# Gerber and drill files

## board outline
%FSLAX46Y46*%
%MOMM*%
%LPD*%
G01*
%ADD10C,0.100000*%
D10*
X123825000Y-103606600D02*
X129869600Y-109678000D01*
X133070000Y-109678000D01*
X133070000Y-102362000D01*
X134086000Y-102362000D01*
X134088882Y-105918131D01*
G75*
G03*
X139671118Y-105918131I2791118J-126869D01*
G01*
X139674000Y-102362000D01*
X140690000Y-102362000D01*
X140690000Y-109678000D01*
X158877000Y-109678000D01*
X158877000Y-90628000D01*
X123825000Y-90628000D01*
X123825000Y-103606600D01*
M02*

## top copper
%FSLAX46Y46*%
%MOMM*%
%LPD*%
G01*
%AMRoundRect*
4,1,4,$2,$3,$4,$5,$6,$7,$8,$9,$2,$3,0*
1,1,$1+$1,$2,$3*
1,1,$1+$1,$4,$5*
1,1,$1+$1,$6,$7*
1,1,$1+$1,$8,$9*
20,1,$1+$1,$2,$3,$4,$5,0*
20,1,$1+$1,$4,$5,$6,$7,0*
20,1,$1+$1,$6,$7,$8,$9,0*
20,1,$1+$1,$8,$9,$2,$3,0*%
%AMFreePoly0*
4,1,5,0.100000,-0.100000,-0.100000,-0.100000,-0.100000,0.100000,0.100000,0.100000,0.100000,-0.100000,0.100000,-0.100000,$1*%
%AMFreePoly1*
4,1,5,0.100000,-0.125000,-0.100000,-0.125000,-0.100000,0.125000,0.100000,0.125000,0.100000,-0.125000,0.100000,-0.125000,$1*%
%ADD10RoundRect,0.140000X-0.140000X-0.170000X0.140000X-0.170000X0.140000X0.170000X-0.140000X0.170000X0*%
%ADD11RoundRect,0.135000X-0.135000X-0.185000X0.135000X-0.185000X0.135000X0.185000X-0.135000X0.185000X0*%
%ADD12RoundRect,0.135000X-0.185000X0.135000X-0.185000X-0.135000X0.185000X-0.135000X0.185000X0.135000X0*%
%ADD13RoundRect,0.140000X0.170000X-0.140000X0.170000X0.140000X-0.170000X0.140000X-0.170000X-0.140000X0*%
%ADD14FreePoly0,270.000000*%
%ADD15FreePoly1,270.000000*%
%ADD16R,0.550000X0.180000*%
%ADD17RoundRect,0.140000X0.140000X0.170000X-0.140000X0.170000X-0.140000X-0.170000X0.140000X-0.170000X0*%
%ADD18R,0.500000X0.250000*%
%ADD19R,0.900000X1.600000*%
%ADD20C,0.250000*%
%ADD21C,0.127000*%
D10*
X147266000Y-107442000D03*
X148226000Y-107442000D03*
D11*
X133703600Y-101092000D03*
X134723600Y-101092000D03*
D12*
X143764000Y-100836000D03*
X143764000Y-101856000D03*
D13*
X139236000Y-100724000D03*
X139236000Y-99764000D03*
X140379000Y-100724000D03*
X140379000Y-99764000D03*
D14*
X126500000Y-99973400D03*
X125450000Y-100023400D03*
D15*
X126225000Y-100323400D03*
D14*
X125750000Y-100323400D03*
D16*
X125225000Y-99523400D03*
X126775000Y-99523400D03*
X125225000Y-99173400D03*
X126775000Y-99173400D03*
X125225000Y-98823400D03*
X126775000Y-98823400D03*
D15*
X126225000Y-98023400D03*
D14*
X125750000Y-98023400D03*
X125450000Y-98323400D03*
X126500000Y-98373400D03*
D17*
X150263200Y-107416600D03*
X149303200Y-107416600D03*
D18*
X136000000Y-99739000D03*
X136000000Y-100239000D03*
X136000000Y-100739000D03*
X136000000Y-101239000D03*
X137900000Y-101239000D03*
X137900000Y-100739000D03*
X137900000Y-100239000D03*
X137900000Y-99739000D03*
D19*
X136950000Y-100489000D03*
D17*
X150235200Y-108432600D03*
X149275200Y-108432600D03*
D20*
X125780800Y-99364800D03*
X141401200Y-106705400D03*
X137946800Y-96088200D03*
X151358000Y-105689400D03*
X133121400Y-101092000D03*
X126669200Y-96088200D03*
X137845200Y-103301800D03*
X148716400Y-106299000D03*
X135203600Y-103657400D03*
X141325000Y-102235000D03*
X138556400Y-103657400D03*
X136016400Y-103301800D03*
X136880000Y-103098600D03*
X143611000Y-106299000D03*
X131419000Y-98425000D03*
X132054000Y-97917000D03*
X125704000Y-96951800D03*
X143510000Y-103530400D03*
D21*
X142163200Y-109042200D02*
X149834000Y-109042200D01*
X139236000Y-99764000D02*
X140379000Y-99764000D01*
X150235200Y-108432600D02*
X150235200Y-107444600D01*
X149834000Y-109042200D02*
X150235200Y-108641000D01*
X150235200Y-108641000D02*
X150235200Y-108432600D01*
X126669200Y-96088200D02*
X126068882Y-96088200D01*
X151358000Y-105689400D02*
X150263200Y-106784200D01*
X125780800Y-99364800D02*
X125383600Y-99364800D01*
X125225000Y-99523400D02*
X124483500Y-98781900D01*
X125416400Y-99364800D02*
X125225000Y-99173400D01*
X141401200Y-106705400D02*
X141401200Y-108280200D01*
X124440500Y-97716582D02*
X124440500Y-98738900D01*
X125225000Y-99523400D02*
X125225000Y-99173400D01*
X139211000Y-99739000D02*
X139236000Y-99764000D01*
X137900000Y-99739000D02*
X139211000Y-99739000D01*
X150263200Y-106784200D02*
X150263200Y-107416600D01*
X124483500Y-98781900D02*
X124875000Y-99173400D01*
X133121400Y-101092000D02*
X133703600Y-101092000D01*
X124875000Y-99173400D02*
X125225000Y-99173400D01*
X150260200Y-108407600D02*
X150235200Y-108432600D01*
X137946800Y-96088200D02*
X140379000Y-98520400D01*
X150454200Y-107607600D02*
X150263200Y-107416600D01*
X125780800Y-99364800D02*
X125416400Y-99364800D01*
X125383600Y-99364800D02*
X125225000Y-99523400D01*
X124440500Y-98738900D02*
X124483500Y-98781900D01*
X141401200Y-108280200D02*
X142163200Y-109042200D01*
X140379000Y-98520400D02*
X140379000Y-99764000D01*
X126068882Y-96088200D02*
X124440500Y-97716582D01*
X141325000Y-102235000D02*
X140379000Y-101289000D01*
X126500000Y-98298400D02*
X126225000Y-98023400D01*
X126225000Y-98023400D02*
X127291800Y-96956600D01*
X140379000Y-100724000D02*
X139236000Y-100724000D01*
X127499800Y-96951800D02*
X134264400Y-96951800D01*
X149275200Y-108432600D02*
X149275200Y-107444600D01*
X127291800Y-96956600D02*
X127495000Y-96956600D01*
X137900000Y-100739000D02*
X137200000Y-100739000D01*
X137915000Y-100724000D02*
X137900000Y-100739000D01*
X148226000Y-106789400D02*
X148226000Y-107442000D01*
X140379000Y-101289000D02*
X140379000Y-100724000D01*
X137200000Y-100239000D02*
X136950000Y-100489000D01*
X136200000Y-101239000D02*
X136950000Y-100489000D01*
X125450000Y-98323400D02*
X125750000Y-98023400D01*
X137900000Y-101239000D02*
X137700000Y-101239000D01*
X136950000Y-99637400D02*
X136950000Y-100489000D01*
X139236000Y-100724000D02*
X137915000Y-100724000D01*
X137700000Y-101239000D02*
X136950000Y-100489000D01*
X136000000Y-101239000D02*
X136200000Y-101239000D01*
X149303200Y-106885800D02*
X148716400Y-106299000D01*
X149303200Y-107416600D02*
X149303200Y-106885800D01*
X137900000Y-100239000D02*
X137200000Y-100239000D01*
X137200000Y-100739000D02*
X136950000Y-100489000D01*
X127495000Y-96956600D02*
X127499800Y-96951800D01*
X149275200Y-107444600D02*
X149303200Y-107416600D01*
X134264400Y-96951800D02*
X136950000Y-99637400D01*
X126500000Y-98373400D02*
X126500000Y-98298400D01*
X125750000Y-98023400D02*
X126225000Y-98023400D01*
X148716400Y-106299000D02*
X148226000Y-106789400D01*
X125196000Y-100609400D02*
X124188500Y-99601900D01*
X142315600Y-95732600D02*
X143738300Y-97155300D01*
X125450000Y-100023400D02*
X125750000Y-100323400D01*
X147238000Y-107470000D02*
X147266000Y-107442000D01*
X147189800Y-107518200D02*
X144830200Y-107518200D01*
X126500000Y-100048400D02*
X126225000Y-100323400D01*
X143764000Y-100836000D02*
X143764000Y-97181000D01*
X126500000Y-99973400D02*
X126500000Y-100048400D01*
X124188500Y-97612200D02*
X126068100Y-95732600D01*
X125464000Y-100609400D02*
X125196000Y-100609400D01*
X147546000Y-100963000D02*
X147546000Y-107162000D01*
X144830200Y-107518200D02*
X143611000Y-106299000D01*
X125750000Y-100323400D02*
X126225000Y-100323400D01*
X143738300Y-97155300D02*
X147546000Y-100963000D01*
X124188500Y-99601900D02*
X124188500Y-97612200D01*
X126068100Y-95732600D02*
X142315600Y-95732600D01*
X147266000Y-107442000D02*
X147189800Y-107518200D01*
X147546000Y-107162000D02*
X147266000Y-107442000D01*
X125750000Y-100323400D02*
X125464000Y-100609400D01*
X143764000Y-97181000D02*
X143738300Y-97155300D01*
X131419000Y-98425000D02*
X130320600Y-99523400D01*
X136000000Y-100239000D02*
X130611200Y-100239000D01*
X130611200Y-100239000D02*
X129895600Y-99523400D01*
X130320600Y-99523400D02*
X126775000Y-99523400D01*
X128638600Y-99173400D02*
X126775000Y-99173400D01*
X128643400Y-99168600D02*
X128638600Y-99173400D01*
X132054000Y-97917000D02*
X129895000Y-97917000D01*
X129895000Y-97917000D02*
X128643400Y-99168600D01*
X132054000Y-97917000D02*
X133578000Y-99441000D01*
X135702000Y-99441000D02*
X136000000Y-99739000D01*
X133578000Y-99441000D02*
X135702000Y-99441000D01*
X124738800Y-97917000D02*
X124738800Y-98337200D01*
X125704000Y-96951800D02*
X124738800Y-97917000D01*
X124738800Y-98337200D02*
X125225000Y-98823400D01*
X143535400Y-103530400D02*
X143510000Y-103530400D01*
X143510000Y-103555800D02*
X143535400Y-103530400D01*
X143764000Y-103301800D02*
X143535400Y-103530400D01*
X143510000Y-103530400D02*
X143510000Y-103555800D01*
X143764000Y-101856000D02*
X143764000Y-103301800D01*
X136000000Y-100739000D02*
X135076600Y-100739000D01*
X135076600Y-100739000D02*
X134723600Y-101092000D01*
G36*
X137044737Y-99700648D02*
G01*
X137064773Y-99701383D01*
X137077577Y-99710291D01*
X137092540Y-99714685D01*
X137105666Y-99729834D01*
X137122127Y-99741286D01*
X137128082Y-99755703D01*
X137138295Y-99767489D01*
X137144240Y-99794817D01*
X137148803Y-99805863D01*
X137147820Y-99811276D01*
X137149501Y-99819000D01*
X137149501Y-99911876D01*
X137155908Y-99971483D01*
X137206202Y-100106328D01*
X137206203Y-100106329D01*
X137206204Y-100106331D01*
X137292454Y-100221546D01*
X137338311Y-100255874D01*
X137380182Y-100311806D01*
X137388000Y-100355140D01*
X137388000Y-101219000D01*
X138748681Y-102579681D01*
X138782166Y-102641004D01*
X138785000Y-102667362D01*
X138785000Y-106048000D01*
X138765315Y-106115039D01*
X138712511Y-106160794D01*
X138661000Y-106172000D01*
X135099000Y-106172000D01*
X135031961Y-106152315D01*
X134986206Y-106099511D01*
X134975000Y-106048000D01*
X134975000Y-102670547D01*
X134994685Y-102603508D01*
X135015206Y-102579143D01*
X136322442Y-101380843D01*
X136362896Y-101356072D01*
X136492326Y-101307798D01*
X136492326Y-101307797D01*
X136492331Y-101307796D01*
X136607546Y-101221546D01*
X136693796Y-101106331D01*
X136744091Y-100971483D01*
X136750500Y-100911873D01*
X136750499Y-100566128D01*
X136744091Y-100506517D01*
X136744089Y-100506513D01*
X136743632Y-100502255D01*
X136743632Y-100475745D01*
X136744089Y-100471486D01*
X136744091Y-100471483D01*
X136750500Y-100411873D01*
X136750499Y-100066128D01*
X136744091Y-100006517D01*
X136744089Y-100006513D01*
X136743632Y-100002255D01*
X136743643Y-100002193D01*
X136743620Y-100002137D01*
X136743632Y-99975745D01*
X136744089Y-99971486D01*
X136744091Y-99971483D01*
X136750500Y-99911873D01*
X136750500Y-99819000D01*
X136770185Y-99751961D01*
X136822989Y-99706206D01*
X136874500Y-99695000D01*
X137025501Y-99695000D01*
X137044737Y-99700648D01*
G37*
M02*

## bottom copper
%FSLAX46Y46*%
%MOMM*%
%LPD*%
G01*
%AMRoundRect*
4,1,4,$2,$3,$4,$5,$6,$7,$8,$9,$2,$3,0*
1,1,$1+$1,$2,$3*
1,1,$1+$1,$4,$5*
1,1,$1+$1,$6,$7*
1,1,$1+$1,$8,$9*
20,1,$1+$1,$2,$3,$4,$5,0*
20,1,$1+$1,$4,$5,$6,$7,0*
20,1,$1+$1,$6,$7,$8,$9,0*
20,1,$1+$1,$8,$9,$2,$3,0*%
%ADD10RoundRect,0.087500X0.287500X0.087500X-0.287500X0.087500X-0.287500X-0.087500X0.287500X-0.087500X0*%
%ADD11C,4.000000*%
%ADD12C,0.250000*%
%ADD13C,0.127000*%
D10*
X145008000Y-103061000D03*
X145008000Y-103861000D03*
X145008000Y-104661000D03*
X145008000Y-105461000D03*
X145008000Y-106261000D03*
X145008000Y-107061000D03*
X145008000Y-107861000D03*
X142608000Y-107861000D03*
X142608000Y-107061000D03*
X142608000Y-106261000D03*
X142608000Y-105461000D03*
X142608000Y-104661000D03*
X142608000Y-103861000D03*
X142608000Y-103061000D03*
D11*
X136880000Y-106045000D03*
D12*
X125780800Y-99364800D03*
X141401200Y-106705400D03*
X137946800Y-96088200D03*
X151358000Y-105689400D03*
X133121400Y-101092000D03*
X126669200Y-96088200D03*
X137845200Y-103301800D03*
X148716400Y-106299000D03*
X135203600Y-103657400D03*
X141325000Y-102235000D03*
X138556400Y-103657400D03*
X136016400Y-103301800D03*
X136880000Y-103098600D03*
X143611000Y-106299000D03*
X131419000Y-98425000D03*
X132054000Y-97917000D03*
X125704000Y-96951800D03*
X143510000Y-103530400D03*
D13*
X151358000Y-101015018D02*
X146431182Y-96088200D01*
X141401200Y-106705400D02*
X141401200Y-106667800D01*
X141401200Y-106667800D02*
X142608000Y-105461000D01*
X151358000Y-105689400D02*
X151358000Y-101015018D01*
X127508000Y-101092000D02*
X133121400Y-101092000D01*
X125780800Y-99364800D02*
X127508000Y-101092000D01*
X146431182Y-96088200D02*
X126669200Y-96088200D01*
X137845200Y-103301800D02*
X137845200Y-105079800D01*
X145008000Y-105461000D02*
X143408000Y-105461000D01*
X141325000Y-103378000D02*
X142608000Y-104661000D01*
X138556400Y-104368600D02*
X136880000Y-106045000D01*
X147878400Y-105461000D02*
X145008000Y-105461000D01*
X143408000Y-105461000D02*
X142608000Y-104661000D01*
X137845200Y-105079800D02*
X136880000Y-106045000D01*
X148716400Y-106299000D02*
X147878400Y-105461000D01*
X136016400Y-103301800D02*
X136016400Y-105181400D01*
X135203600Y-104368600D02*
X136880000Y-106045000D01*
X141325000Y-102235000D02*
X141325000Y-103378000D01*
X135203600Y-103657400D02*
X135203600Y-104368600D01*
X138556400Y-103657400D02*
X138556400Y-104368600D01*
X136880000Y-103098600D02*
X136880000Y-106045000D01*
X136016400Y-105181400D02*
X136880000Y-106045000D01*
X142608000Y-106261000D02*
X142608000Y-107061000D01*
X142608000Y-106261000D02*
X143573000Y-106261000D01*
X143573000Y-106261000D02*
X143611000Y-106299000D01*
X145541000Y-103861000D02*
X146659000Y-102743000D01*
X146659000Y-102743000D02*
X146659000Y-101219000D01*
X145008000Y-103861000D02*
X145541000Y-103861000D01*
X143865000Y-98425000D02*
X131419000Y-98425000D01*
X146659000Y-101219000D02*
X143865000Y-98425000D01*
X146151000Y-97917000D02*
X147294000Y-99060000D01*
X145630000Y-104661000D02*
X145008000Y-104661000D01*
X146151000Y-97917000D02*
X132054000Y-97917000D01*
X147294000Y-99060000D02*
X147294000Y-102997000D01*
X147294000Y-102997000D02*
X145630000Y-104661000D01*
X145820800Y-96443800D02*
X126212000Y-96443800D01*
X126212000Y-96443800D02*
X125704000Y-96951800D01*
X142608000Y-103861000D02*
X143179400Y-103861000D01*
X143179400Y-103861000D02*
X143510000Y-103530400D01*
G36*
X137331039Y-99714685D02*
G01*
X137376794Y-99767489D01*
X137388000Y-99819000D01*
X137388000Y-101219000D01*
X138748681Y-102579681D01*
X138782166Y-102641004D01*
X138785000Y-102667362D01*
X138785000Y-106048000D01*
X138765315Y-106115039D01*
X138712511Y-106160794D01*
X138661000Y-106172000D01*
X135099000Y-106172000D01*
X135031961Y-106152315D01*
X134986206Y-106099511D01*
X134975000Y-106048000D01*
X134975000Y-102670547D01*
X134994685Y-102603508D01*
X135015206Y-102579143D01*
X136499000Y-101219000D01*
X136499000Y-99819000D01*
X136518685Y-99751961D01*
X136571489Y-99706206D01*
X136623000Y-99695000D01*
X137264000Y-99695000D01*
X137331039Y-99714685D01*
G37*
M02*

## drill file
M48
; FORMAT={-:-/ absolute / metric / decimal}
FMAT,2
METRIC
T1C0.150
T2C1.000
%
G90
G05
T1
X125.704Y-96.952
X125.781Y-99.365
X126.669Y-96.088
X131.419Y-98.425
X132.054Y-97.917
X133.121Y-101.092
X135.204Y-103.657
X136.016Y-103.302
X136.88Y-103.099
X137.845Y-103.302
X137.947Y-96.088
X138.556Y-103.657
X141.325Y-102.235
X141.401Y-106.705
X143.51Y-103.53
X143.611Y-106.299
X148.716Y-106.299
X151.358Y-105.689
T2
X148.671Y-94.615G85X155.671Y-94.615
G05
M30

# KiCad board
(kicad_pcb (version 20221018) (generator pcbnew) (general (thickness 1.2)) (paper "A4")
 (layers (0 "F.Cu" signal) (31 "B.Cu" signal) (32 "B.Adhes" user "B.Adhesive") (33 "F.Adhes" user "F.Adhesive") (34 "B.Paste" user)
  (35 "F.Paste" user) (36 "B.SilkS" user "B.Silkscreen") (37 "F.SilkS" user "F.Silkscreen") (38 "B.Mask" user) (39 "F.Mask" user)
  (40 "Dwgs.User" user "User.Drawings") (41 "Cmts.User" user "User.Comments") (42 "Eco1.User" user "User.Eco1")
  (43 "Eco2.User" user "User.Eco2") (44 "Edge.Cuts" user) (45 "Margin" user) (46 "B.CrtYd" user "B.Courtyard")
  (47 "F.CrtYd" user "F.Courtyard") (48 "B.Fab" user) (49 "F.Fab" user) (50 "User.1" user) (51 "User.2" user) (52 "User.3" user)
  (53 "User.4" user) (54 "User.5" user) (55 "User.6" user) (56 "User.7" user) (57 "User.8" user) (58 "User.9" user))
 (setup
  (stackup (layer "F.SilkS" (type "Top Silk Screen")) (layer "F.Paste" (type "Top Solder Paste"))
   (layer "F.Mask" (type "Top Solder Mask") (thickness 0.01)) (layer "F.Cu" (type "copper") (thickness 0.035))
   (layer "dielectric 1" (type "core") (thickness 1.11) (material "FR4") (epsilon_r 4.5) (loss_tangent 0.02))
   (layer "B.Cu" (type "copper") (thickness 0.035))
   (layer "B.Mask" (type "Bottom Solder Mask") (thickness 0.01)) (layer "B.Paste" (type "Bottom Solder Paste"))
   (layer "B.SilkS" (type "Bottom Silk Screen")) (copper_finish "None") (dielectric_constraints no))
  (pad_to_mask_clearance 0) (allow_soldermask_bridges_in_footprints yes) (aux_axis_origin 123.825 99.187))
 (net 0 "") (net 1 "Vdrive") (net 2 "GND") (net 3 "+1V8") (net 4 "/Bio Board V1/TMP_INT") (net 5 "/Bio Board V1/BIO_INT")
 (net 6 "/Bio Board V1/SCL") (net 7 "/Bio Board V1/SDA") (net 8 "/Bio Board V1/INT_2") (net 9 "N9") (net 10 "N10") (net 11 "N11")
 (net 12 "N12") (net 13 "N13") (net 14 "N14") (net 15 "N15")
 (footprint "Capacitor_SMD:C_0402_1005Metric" (layer "F.Cu") (at 147.746 107.442)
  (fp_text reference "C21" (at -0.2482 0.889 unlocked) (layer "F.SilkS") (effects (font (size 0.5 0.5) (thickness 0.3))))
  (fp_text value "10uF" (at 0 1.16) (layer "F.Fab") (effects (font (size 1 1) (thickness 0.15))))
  (pad "1" smd roundrect (at -0.48 0) (size 0.56 0.62) (layers "F.Cu" "F.Paste" "F.Mask") (roundrect_rratio 0.25) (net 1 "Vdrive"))
  (pad "2" smd roundrect (at 0.48 0) (size 0.56 0.62) (layers "F.Cu" "F.Paste" "F.Mask") (roundrect_rratio 0.25) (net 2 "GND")))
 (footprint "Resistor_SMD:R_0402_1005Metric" (layer "F.Cu") (at 134.2136 101.092)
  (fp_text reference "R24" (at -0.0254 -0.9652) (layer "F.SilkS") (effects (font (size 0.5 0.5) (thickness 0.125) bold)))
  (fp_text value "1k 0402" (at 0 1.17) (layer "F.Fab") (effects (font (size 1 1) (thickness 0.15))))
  (pad "1" smd roundrect (at -0.51 0) (size 0.54 0.64) (layers "F.Cu" "F.Paste" "F.Mask") (roundrect_rratio 0.25) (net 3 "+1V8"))
  (pad "2" smd roundrect (at 0.51 0) (size 0.54 0.64) (layers "F.Cu" "F.Paste" "F.Mask") (roundrect_rratio 0.25)
   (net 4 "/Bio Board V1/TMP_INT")))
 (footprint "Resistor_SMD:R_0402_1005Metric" (layer "F.Cu") (at 143.764 101.346 -90)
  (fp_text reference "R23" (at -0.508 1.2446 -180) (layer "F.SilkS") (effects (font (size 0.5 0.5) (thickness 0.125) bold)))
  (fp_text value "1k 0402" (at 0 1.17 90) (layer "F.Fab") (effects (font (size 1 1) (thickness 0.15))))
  (pad "1" smd roundrect (at -0.51 0 270) (size 0.54 0.64) (layers "F.Cu" "F.Paste" "F.Mask") (roundrect_rratio 0.25) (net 1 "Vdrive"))
  (pad "2" smd roundrect (at 0.51 0 270) (size 0.54 0.64) (layers "F.Cu" "F.Paste" "F.Mask") (roundrect_rratio 0.25)
   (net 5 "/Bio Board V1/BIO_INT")))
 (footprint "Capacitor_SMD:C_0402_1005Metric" (layer "F.Cu") (at 139.236 100.244 90)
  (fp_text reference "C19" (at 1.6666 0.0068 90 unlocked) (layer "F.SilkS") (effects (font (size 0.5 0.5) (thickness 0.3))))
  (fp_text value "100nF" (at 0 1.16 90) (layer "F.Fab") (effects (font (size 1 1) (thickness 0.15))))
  (pad "1" smd roundrect (at -0.48 0 90) (size 0.56 0.62) (layers "F.Cu" "F.Paste" "F.Mask") (roundrect_rratio 0.25) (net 2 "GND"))
  (pad "2" smd roundrect (at 0.48 0 90) (size 0.56 0.62) (layers "F.Cu" "F.Paste" "F.Mask") (roundrect_rratio 0.25) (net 3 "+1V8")))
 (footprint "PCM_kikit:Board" (layer "F.Cu") (at 144.8048 90.6018)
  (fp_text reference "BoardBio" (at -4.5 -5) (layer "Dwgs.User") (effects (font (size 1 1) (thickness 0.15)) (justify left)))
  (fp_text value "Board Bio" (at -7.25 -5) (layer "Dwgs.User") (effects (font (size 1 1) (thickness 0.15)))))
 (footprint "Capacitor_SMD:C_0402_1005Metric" (layer "F.Cu") (at 140.379 100.244 90)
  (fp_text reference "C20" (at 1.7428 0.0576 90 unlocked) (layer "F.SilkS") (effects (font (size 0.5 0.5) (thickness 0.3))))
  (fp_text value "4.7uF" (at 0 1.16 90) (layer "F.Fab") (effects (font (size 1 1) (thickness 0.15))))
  (pad "1" smd roundrect (at -0.48 0 90) (size 0.56 0.62) (layers "F.Cu" "F.Paste" "F.Mask") (roundrect_rratio 0.25) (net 2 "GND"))
  (pad "2" smd roundrect (at 0.48 0 90) (size 0.56 0.62) (layers "F.Cu" "F.Paste" "F.Mask") (roundrect_rratio 0.25) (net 3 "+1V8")))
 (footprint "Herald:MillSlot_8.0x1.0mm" (layer "F.Cu") (at 152.1708 94.615)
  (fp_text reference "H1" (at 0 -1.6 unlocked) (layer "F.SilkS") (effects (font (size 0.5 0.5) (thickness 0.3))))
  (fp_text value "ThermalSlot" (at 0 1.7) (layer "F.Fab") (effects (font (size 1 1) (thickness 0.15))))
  (pad "" np_thru_hole oval (at 0 0) (size 8 1) (drill oval 8 1) (layers "F&B.Cu" "*.Mask")))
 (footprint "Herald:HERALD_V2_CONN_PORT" (layer "F.Cu") (at 126 99.1734 -90)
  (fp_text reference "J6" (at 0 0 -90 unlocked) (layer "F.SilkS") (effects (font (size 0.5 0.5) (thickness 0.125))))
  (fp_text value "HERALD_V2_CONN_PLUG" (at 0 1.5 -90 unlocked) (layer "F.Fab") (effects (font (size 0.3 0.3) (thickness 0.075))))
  (pad "1" smd custom (at 0.8 -0.5 270) (size 0.2 0.2) (layers "F.Cu" "F.Paste" "F.Mask") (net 1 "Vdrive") (thermal_bridge_angle 45)
   (options (clearance outline) (anchor rect)) (primitives))
  (pad "1" smd custom (at 0.85 0.55 270) (size 0.2 0.2) (layers "F.Cu" "F.Paste" "F.Mask") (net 1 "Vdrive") (thermal_bridge_angle 45)
   (options (clearance outline) (anchor rect)) (primitives))
  (pad "1" smd custom (at 1.15 -0.225 270) (size 0.2 0.25) (layers "F.Cu" "F.Paste" "F.Mask") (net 1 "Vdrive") (thermal_bridge_angle 45)
   (options (clearance outline) (anchor rect)) (primitives))
  (pad "1" smd custom (at 1.15 0.25 270) (size 0.2 0.2) (layers "F.Cu" "F.Paste" "F.Mask") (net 1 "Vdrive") (thermal_bridge_angle 45)
   (options (clearance outline) (anchor rect)) (primitives))
  (pad "2" smd rect (at 0.35 0.775 270) (size 0.18 0.55) (layers "F.Cu" "F.Paste" "F.Mask") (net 3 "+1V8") (thermal_bridge_angle 45))
  (pad "3" smd rect (at 0.35 -0.775 270) (size 0.18 0.55) (layers "F.Cu" "F.Paste" "F.Mask") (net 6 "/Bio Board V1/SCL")
   (thermal_bridge_angle 45))
  (pad "4" smd rect (at 0 0.775 270) (size 0.18 0.55) (layers "F.Cu" "F.Paste" "F.Mask") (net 3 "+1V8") (thermal_bridge_angle 45))
  (pad "5" smd rect (at 0 -0.775 270) (size 0.18 0.55) (layers "F.Cu" "F.Paste" "F.Mask") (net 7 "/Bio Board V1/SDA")
   (thermal_bridge_angle 45))
  (pad "6" smd rect (at -0.35 0.775 270) (size 0.18 0.55) (layers "F.Cu" "F.Paste" "F.Mask") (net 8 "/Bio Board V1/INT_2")
   (thermal_bridge_angle 45))
  (pad "7" smd rect (at -0.35 -0.775 270) (size 0.18 0.55) (layers "F.Cu" "F.Paste" "F.Mask") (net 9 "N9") (thermal_bridge_angle 45))
  (pad "8" smd custom (at -1.15 -0.225 270) (size 0.2 0.25) (layers "F.Cu" "F.Paste" "F.Mask") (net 2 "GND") (thermal_bridge_angle 45)
   (options (clearance outline) (anchor rect)) (primitives))
  (pad "8" smd custom (at -1.15 0.25 270) (size 0.2 0.2) (layers "F.Cu" "F.Paste" "F.Mask") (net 2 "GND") (thermal_bridge_angle 45)
   (options (clearance outline) (anchor rect)) (primitives))
  (pad "8" smd custom (at -0.85 0.55 270) (size 0.2 0.2) (layers "F.Cu" "F.Paste" "F.Mask") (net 2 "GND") (thermal_bridge_angle 45)
   (options (clearance outline) (anchor rect)) (primitives))
  (pad "8" smd custom (at -0.8 -0.5 270) (size 0.2 0.2) (layers "F.Cu" "F.Paste" "F.Mask") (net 2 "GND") (thermal_bridge_angle 45)
   (options (clearance outline) (anchor rect)) (primitives)))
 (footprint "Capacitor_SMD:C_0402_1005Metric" (layer "F.Cu") (at 149.7832 107.4166 180)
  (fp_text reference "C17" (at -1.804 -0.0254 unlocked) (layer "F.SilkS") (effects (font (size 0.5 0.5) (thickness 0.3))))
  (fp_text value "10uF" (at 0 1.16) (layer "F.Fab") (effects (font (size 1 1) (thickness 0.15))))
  (pad "1" smd roundrect (at -0.48 0 180) (size 0.56 0.62) (layers "F.Cu" "F.Paste" "F.Mask") (roundrect_rratio 0.25) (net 3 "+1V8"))
  (pad "2" smd roundrect (at 0.48 0 180) (size 0.56 0.62) (layers "F.Cu" "F.Paste" "F.Mask") (roundrect_rratio 0.25) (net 2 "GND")))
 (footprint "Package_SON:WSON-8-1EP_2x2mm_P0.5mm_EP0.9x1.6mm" (layer "F.Cu") (at 136.95 100.489)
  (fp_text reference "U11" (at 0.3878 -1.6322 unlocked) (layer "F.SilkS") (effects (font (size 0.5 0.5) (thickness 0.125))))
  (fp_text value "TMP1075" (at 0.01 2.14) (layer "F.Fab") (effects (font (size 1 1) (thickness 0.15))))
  (pad "" smd rect (at 0 -0.4) (size 0.75 0.65) (layers "F.Paste"))
  (pad "" smd rect (at 0 0.4) (size 0.75 0.65) (layers "F.Paste"))
  (pad "1" smd rect (at -0.95 -0.75) (size 0.5 0.25) (layers "F.Cu" "F.Paste" "F.Mask") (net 7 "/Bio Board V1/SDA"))
  (pad "2" smd rect (at -0.95 -0.25) (size 0.5 0.25) (layers "F.Cu" "F.Paste" "F.Mask") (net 6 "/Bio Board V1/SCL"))
  (pad "3" smd rect (at -0.95 0.25) (size 0.5 0.25) (layers "F.Cu" "F.Paste" "F.Mask") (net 4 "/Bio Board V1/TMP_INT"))
  (pad "4" smd rect (at -0.95 0.75) (size 0.5 0.25) (layers "F.Cu" "F.Paste" "F.Mask") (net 2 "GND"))
  (pad "5" smd rect (at 0.95 0.75) (size 0.5 0.25) (layers "F.Cu" "F.Paste" "F.Mask") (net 2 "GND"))
  (pad "6" smd rect (at 0.95 0.25) (size 0.5 0.25) (layers "F.Cu" "F.Paste" "F.Mask") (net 2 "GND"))
  (pad "7" smd rect (at 0.95 -0.25) (size 0.5 0.25) (layers "F.Cu" "F.Paste" "F.Mask") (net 2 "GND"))
  (pad "8" smd rect (at 0.95 -0.75) (size 0.5 0.25) (layers "F.Cu" "F.Paste" "F.Mask") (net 3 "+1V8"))
  (pad "9" smd rect (at 0 0) (size 0.9 1.6) (layers "F.Cu" "F.Mask") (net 2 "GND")))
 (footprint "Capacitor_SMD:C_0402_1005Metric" (layer "F.Cu") (at 149.7552 108.4326 180)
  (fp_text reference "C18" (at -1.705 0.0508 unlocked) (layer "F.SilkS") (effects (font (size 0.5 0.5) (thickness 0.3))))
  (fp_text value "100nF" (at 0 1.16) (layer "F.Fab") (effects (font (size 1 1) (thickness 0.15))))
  (pad "1" smd roundrect (at -0.48 0 180) (size 0.56 0.62) (layers "F.Cu" "F.Paste" "F.Mask") (roundrect_rratio 0.25) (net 3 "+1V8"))
  (pad "2" smd roundrect (at 0.48 0 180) (size 0.56 0.62) (layers "F.Cu" "F.Paste" "F.Mask") (roundrect_rratio 0.25) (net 2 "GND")))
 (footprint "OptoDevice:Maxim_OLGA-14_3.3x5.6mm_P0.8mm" (layer "B.Cu") (at 143.808 105.461 180)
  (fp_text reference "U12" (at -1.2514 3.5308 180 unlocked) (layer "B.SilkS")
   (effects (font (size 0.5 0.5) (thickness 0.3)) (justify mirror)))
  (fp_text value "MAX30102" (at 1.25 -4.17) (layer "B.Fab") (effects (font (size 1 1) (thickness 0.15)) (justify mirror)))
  (pad "1" smd roundrect (at -1.2 2.4 180) (size 0.75 0.35) (layers "B.Cu" "B.Paste" "B.Mask") (roundrect_rratio 0.25) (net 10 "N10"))
  (pad "2" smd roundrect (at -1.2 1.6 180) (size 0.75 0.35) (layers "B.Cu" "B.Paste" "B.Mask") (roundrect_rratio 0.25)
   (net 6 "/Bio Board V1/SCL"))
  (pad "3" smd roundrect (at -1.2 0.8 180) (size 0.75 0.35) (layers "B.Cu" "B.Paste" "B.Mask") (roundrect_rratio 0.25)
   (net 7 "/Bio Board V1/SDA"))
  (pad "4" smd roundrect (at -1.2 0 180) (size 0.75 0.35) (layers "B.Cu" "B.Paste" "B.Mask") (roundrect_rratio 0.25) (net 2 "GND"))
  (pad "5" smd roundrect (at -1.2 -0.8 180) (size 0.75 0.35) (layers "B.Cu" "B.Paste" "B.Mask") (roundrect_rratio 0.25) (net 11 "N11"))
  (pad "6" smd roundrect (at -1.2 -1.6 180) (size 0.75 0.35) (layers "B.Cu" "B.Paste" "B.Mask") (roundrect_rratio 0.25) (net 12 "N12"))
  (pad "7" smd roundrect (at -1.2 -2.4 180) (size 0.75 0.35) (layers "B.Cu" "B.Paste" "B.Mask") (roundrect_rratio 0.25) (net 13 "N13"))
  (pad "8" smd roundrect (at 1.2 -2.4 180) (size 0.75 0.35) (layers "B.Cu" "B.Paste" "B.Mask") (roundrect_rratio 0.25) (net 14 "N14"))
  (pad "9" smd roundrect (at 1.2 -1.6 180) (size 0.75 0.35) (layers "B.Cu" "B.Paste" "B.Mask") (roundrect_rratio 0.25) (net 1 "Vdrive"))
  (pad "10" smd roundrect (at 1.2 -0.8 180) (size 0.75 0.35) (layers "B.Cu" "B.Paste" "B.Mask") (roundrect_rratio 0.25) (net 1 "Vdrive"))
  (pad "11" smd roundrect (at 1.2 0 180) (size 0.75 0.35) (layers "B.Cu" "B.Paste" "B.Mask") (roundrect_rratio 0.25) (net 3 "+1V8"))
  (pad "12" smd roundrect (at 1.2 0.8 180) (size 0.75 0.35) (layers "B.Cu" "B.Paste" "B.Mask") (roundrect_rratio 0.25) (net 2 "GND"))
  (pad "13" smd roundrect (at 1.2 1.6 180) (size 0.75 0.35) (layers "B.Cu" "B.Paste" "B.Mask") (roundrect_rratio 0.25)
   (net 5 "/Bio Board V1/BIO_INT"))
  (pad "14" smd roundrect (at 1.2 2.4 180) (size 0.75 0.35) (layers "B.Cu" "B.Paste" "B.Mask") (roundrect_rratio 0.25) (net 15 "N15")))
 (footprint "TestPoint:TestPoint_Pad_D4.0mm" (layer "B.Cu") (at 136.88 106.045 180)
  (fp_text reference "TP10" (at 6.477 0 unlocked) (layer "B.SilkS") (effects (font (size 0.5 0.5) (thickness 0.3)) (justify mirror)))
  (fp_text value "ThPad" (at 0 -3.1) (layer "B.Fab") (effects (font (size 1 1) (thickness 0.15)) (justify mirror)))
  (pad "1" smd circle (at 0 0 180) (size 4 4) (layers "B.Cu" "B.Mask") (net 2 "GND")))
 (gr_poly
  (pts (xy 123.825 103.6066) (xy 129.8696 109.678) (xy 133.07 109.678) (xy 133.07 102.362) (xy 134.086 102.362)
   (arc (start 134.088882 105.918131) (mid 136.88 108.839) (end 139.671118 105.918131)) (xy 139.674 102.362) (xy 140.69 102.362)
   (xy 140.69 109.678) (xy 158.877 109.678) (xy 158.877 90.628) (xy 123.825 90.628))
  (stroke (width 0.1) (type solid)) (fill none) (layer "Edge.Cuts"))
 (segment (start 142.1632 109.0422) (end 149.834 109.0422) (width 0.127) (layer "F.Cu") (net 3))
 (segment (start 139.236 99.764) (end 140.379 99.764) (width 0.127) (layer "F.Cu") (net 3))
 (segment (start 150.2352 108.4326) (end 150.2352 107.4446) (width 0.127) (layer "F.Cu") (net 3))
 (segment (start 149.834 109.0422) (end 150.2352 108.641) (width 0.127) (layer "F.Cu") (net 3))
 (segment (start 150.2352 108.641) (end 150.2352 108.4326) (width 0.127) (layer "F.Cu") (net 3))
 (segment (start 126.6692 96.0882) (end 126.068882 96.0882) (width 0.127) (layer "F.Cu") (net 3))
 (segment (start 151.358 105.6894) (end 150.2632 106.7842) (width 0.127) (layer "F.Cu") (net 3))
 (segment (start 125.7808 99.3648) (end 125.3836 99.3648) (width 0.127) (layer "F.Cu") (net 3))
 (segment (start 125.225 99.5234) (end 124.4835 98.7819) (width 0.127) (layer "F.Cu") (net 3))
 (segment (start 125.4164 99.3648) (end 125.225 99.1734) (width 0.127) (layer "F.Cu") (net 3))
 (segment (start 141.4012 106.7054) (end 141.4012 108.2802) (width 0.127) (layer "F.Cu") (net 3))
 (segment (start 124.4405 97.716582) (end 124.4405 98.7389) (width 0.127) (layer "F.Cu") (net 3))
 (segment (start 125.225 99.5234) (end 125.225 99.1734) (width 0.127) (layer "F.Cu") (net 3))
 (segment (start 139.211 99.739) (end 139.236 99.764) (width 0.127) (layer "F.Cu") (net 3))
 (segment (start 137.9 99.739) (end 139.211 99.739) (width 0.127) (layer "F.Cu") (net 3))
 (segment (start 150.2632 106.7842) (end 150.2632 107.4166) (width 0.127) (layer "F.Cu") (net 3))
 (segment (start 124.4835 98.7819) (end 124.875 99.1734) (width 0.127) (layer "F.Cu") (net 3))
 (segment (start 133.1214 101.092) (end 133.7036 101.092) (width 0.127) (layer "F.Cu") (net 3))
 (segment (start 124.875 99.1734) (end 125.225 99.1734) (width 0.127) (layer "F.Cu") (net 3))
 (segment (start 150.2602 108.4076) (end 150.2352 108.4326) (width 0.127) (layer "F.Cu") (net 3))
 (segment (start 137.9468 96.0882) (end 140.379 98.5204) (width 0.127) (layer "F.Cu") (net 3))
 (segment (start 150.4542 107.6076) (end 150.2632 107.4166) (width 0.127) (layer "F.Cu") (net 3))
 (segment (start 125.7808 99.3648) (end 125.4164 99.3648) (width 0.127) (layer "F.Cu") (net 3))
 (segment (start 125.3836 99.3648) (end 125.225 99.5234) (width 0.127) (layer "F.Cu") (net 3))
 (segment (start 124.4405 98.7389) (end 124.4835 98.7819) (width 0.127) (layer "F.Cu") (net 3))
 (segment (start 141.4012 108.2802) (end 142.1632 109.0422) (width 0.127) (layer "F.Cu") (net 3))
 (segment (start 140.379 98.5204) (end 140.379 99.764) (width 0.127) (layer "F.Cu") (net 3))
 (segment (start 126.068882 96.0882) (end 124.4405 97.716582) (width 0.127) (layer "F.Cu") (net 3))
 (via (at 125.7808 99.3648) (size 0.25) (drill 0.15) (layers "F.Cu" "B.Cu") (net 3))
 (via (at 141.4012 106.7054) (size 0.25) (drill 0.15) (layers "F.Cu" "B.Cu") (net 3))
 (via (at 137.9468 96.0882) (size 0.25) (drill 0.15) (layers "F.Cu" "B.Cu") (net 3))
 (via (at 151.358 105.6894) (size 0.25) (drill 0.15) (layers "F.Cu" "B.Cu") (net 3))
 (via (at 133.1214 101.092) (size 0.25) (drill 0.15) (layers "F.Cu" "B.Cu") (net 3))
 (via (at 126.6692 96.0882) (size 0.25) (drill 0.15) (layers "F.Cu" "B.Cu") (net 3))
 (segment (start 151.358 101.015018) (end 146.431182 96.0882) (width 0.127) (layer "B.Cu") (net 3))
 (segment (start 141.4012 106.7054) (end 141.4012 106.6678) (width 0.127) (layer "B.Cu") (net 3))
 (segment (start 141.4012 106.6678) (end 142.608 105.461) (width 0.127) (layer "B.Cu") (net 3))
 (segment (start 151.358 105.6894) (end 151.358 101.015018) (width 0.127) (layer "B.Cu") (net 3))
 (segment (start 127.508 101.092) (end 133.1214 101.092) (width 0.127) (layer "B.Cu") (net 3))
 (segment (start 125.7808 99.3648) (end 127.508 101.092) (width 0.127) (layer "B.Cu") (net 3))
 (segment (start 146.431182 96.0882) (end 126.6692 96.0882) (width 0.127) (layer "B.Cu") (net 3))
 (segment (start 141.325 102.235) (end 140.379 101.289) (width 0.127) (layer "F.Cu") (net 2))
 (segment (start 126.5 98.2984) (end 126.225 98.0234) (width 0.127) (layer "F.Cu") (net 2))
 (segment (start 126.225 98.0234) (end 127.2918 96.9566) (width 0.127) (layer "F.Cu") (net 2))
 (segment (start 140.379 100.724) (end 139.236 100.724) (width 0.127) (layer "F.Cu") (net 2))
 (segment (start 127.4998 96.9518) (end 134.2644 96.9518) (width 0.127) (layer "F.Cu") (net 2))
 (segment (start 149.2752 108.4326) (end 149.2752 107.4446) (width 0.127) (layer "F.Cu") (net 2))
 (segment (start 127.2918 96.9566) (end 127.495 96.9566) (width 0.127) (layer "F.Cu") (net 2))
 (segment (start 137.9 100.739) (end 137.2 100.739) (width 0.127) (layer "F.Cu") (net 2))
 (segment (start 137.915 100.724) (end 137.9 100.739) (width 0.127) (layer "F.Cu") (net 2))
 (segment (start 148.226 106.7894) (end 148.226 107.442) (width 0.127) (layer "F.Cu") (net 2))
 (segment (start 140.379 101.289) (end 140.379 100.724) (width 0.127) (layer "F.Cu") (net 2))
 (segment (start 137.2 100.239) (end 136.95 100.489) (width 0.127) (layer "F.Cu") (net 2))
 (segment (start 136.2 101.239) (end 136.95 100.489) (width 0.127) (layer "F.Cu") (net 2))
 (segment (start 125.45 98.3234) (end 125.75 98.0234) (width 0.127) (layer "F.Cu") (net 2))
 (segment (start 137.9 101.239) (end 137.7 101.239) (width 0.127) (layer "F.Cu") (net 2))
 (segment (start 136.95 99.6374) (end 136.95 100.489) (width 0.127) (layer "F.Cu") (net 2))
 (segment (start 139.236 100.724) (end 137.915 100.724) (width 0.127) (layer "F.Cu") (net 2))
 (segment (start 137.7 101.239) (end 136.95 100.489) (width 0.127) (layer "F.Cu") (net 2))
 (segment (start 136 101.239) (end 136.2 101.239) (width 0.127) (layer "F.Cu") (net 2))
 (segment (start 149.3032 106.8858) (end 148.7164 106.299) (width 0.127) (layer "F.Cu") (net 2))
 (segment (start 149.3032 107.4166) (end 149.3032 106.8858) (width 0.127) (layer "F.Cu") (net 2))
 (segment (start 137.9 100.239) (end 137.2 100.239) (width 0.127) (layer "F.Cu") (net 2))
 (segment (start 137.2 100.739) (end 136.95 100.489) (width 0.127) (layer "F.Cu") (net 2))
 (segment (start 127.495 96.9566) (end 127.4998 96.9518) (width 0.127) (layer "F.Cu") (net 2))
 (segment (start 149.2752 107.4446) (end 149.3032 107.4166) (width 0.127) (layer "F.Cu") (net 2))
 (segment (start 134.2644 96.9518) (end 136.95 99.6374) (width 0.127) (layer "F.Cu") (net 2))
 (segment (start 126.5 98.3734) (end 126.5 98.2984) (width 0.127) (layer "F.Cu") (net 2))
 (segment (start 125.75 98.0234) (end 126.225 98.0234) (width 0.127) (layer "F.Cu") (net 2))
 (segment (start 148.7164 106.299) (end 148.226 106.7894) (width 0.127) (layer "F.Cu") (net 2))
 (via (at 137.8452 103.3018) (size 0.25) (drill 0.15) (layers "F.Cu" "B.Cu") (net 2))
 (via (at 148.7164 106.299) (size 0.25) (drill 0.15) (layers "F.Cu" "B.Cu") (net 2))
 (via (at 135.2036 103.6574) (size 0.25) (drill 0.15) (layers "F.Cu" "B.Cu") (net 2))
 (via (at 141.325 102.235) (size 0.25) (drill 0.15) (layers "F.Cu" "B.Cu") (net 2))
 (via (at 138.5564 103.6574) (size 0.25) (drill 0.15) (layers "F.Cu" "B.Cu") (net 2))
 (via (at 136.0164 103.3018) (size 0.25) (drill 0.15) (layers "F.Cu" "B.Cu") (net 2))
 (via (at 136.88 103.0986) (size 0.25) (drill 0.15) (layers "F.Cu" "B.Cu") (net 2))
 (segment (start 137.8452 103.3018) (end 137.8452 105.0798) (width 0.127) (layer "B.Cu") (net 2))
 (segment (start 145.008 105.461) (end 143.408 105.461) (width 0.127) (layer "B.Cu") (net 2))
 (segment (start 141.325 103.378) (end 142.608 104.661) (width 0.127) (layer "B.Cu") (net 2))
 (segment (start 138.5564 104.3686) (end 136.88 106.045) (width 0.127) (layer "B.Cu") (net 2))
 (segment (start 147.8784 105.461) (end 145.008 105.461) (width 0.127) (layer "B.Cu") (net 2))
 (segment (start 143.408 105.461) (end 142.608 104.661) (width 0.127) (layer "B.Cu") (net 2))
 (segment (start 137.8452 105.0798) (end 136.88 106.045) (width 0.127) (layer "B.Cu") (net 2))
 (segment (start 148.7164 106.299) (end 147.8784 105.461) (width 0.127) (layer "B.Cu") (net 2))
 (segment (start 136.0164 103.3018) (end 136.0164 105.1814) (width 0.127) (layer "B.Cu") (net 2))
 (segment (start 135.2036 104.3686) (end 136.88 106.045) (width 0.127) (layer "B.Cu") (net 2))
 (segment (start 141.325 102.235) (end 141.325 103.378) (width 0.127) (layer "B.Cu") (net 2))
 (segment (start 135.2036 103.6574) (end 135.2036 104.3686) (width 0.127) (layer "B.Cu") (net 2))
 (segment (start 138.5564 103.6574) (end 138.5564 104.3686) (width 0.127) (layer "B.Cu") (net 2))
 (segment (start 136.88 103.0986) (end 136.88 106.045) (width 0.127) (layer "B.Cu") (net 2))
 (segment (start 136.0164 105.1814) (end 136.88 106.045) (width 0.127) (layer "B.Cu") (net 2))
 (segment (start 125.196 100.6094) (end 124.1885 99.6019) (width 0.127) (layer "F.Cu") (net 1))
 (segment (start 142.3156 95.7326) (end 143.7383 97.1553) (width 0.127) (layer "F.Cu") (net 1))
 (segment (start 125.45 100.0234) (end 125.75 100.3234) (width 0.127) (layer "F.Cu") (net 1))
 (segment (start 147.238 107.47) (end 147.266 107.442) (width 0.127) (layer "F.Cu") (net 1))
 (segment (start 147.1898 107.5182) (end 144.8302 107.5182) (width 0.127) (layer "F.Cu") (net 1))
 (segment (start 126.5 100.0484) (end 126.225 100.3234) (width 0.127) (layer "F.Cu") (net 1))
 (segment (start 143.764 100.836) (end 143.764 97.181) (width 0.127) (layer "F.Cu") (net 1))
 (segment (start 126.5 99.9734) (end 126.5 100.0484) (width 0.127) (layer "F.Cu") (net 1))
 (segment (start 124.1885 97.6122) (end 126.0681 95.7326) (width 0.127) (layer "F.Cu") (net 1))
 (segment (start 125.464 100.6094) (end 125.196 100.6094) (width 0.127) (layer "F.Cu") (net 1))
 (segment (start 147.546 100.963) (end 147.546 107.162) (width 0.127) (layer "F.Cu") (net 1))
 (segment (start 144.8302 107.5182) (end 143.611 106.299) (width 0.127) (layer "F.Cu") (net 1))
 (segment (start 125.75 100.3234) (end 126.225 100.3234) (width 0.127) (layer "F.Cu") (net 1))
 (segment (start 143.7383 97.1553) (end 147.546 100.963) (width 0.127) (layer "F.Cu") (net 1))
 (segment (start 124.1885 99.6019) (end 124.1885 97.6122) (width 0.127) (layer "F.Cu") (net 1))
 (segment (start 126.0681 95.7326) (end 142.3156 95.7326) (width 0.127) (layer "F.Cu") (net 1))
 (segment (start 147.266 107.442) (end 147.1898 107.5182) (width 0.127) (layer "F.Cu") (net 1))
 (segment (start 147.546 107.162) (end 147.266 107.442) (width 0.127) (layer "F.Cu") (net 1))
 (segment (start 125.75 100.3234) (end 125.464 100.6094) (width 0.127) (layer "F.Cu") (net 1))
 (segment (start 143.764 97.181) (end 143.7383 97.1553) (width 0.127) (layer "F.Cu") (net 1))
 (via (at 143.611 106.299) (size 0.25) (drill 0.15) (layers "F.Cu" "B.Cu") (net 1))
 (segment (start 142.608 106.261) (end 142.608 107.061) (width 0.127) (layer "B.Cu") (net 1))
 (segment (start 142.608 106.261) (end 143.573 106.261) (width 0.127) (layer "B.Cu") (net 1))
 (segment (start 143.573 106.261) (end 143.611 106.299) (width 0.127) (layer "B.Cu") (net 1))
 (segment (start 131.419 98.425) (end 130.3206 99.5234) (width 0.127) (layer "F.Cu") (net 6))
 (segment (start 136 100.239) (end 130.6112 100.239) (width 0.127) (layer "F.Cu") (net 6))
 (segment (start 130.6112 100.239) (end 129.8956 99.5234) (width 0.127) (layer "F.Cu") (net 6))
 (segment (start 130.3206 99.5234) (end 126.775 99.5234) (width 0.127) (layer "F.Cu") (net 6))
 (via (at 131.419 98.425) (size 0.25) (drill 0.15) (layers "F.Cu" "B.Cu") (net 6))
 (segment (start 145.541 103.861) (end 146.659 102.743) (width 0.127) (layer "B.Cu") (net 6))
 (segment (start 146.659 102.743) (end 146.659 101.219) (width 0.127) (layer "B.Cu") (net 6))
 (segment (start 145.008 103.861) (end 145.541 103.861) (width 0.127) (layer "B.Cu") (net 6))
 (segment (start 143.865 98.425) (end 131.419 98.425) (width 0.127) (layer "B.Cu") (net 6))
 (segment (start 146.659 101.219) (end 143.865 98.425) (width 0.127) (layer "B.Cu") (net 6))
 (segment (start 128.6386 99.1734) (end 126.775 99.1734) (width 0.127) (layer "F.Cu") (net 7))
 (segment (start 128.6434 99.1686) (end 128.6386 99.1734) (width 0.127) (layer "F.Cu") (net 7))
 (segment (start 132.054 97.917) (end 129.895 97.917) (width 0.127) (layer "F.Cu") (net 7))
 (segment (start 129.895 97.917) (end 128.6434 99.1686) (width 0.127) (layer "F.Cu") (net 7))
 (segment (start 132.054 97.917) (end 133.578 99.441) (width 0.127) (layer "F.Cu") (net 7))
 (segment (start 135.702 99.441) (end 136 99.739) (width 0.127) (layer "F.Cu") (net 7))
 (segment (start 133.578 99.441) (end 135.702 99.441) (width 0.127) (layer "F.Cu") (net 7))
 (via (at 132.054 97.917) (size 0.25) (drill 0.15) (layers "F.Cu" "B.Cu") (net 7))
 (segment (start 146.151 97.917) (end 147.294 99.06) (width 0.127) (layer "B.Cu") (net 7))
 (segment (start 145.63 104.661) (end 145.008 104.661) (width 0.127) (layer "B.Cu") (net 7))
 (segment (start 146.151 97.917) (end 132.054 97.917) (width 0.127) (layer "B.Cu") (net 7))
 (segment (start 147.294 99.06) (end 147.294 102.997) (width 0.127) (layer "B.Cu") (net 7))
 (segment (start 147.294 102.997) (end 145.63 104.661) (width 0.127) (layer "B.Cu") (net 7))
 (segment (start 124.7388 97.917) (end 124.7388 98.3372) (width 0.127) (layer "F.Cu") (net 8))
 (segment (start 125.704 96.9518) (end 124.7388 97.917) (width 0.127) (layer "F.Cu") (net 8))
 (segment (start 124.7388 98.3372) (end 125.225 98.8234) (width 0.127) (layer "F.Cu") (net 8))
 (via (at 125.704 96.9518) (size 0.25) (drill 0.15) (layers "F.Cu" "B.Cu") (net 8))
 (segment (start 145.8208 96.4438) (end 126.212 96.4438) (width 0.127) (layer "B.Cu") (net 8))
 (segment (start 126.212 96.4438) (end 125.704 96.9518) (width 0.127) (layer "B.Cu") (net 8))
 (segment (start 143.5354 103.5304) (end 143.51 103.5304) (width 0.127) (layer "F.Cu") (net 5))
 (segment (start 143.51 103.5558) (end 143.5354 103.5304) (width 0.127) (layer "F.Cu") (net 5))
 (segment (start 143.764 103.3018) (end 143.5354 103.5304) (width 0.127) (layer "F.Cu") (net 5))
 (segment (start 143.51 103.5304) (end 143.51 103.5558) (width 0.127) (layer "F.Cu") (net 5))
 (segment (start 143.764 101.856) (end 143.764 103.3018) (width 0.127) (layer "F.Cu") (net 5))
 (via (at 143.51 103.5304) (size 0.25) (drill 0.15) (layers "F.Cu" "B.Cu") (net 5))
 (segment (start 142.608 103.861) (end 143.1794 103.861) (width 0.127) (layer "B.Cu") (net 5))
 (segment (start 143.1794 103.861) (end 143.51 103.5304) (width 0.127) (layer "B.Cu") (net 5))
 (segment (start 136 100.739) (end 135.0766 100.739) (width 0.127) (layer "F.Cu") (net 4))
 (segment (start 135.0766 100.739) (end 134.7236 101.092) (width 0.127) (layer "F.Cu") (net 4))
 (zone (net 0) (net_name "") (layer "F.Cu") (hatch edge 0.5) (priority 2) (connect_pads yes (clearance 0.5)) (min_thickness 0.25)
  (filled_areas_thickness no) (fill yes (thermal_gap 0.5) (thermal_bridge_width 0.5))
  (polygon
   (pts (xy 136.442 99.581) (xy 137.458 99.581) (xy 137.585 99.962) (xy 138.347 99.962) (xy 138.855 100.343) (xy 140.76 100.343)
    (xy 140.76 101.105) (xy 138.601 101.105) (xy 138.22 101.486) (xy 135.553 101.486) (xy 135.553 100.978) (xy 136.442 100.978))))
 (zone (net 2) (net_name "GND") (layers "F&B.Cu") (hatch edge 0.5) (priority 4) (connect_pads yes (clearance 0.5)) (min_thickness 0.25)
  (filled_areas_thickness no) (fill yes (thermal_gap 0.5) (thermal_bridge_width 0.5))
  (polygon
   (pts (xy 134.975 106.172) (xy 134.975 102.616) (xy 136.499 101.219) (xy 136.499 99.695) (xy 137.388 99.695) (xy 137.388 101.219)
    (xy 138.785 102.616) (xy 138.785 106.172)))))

